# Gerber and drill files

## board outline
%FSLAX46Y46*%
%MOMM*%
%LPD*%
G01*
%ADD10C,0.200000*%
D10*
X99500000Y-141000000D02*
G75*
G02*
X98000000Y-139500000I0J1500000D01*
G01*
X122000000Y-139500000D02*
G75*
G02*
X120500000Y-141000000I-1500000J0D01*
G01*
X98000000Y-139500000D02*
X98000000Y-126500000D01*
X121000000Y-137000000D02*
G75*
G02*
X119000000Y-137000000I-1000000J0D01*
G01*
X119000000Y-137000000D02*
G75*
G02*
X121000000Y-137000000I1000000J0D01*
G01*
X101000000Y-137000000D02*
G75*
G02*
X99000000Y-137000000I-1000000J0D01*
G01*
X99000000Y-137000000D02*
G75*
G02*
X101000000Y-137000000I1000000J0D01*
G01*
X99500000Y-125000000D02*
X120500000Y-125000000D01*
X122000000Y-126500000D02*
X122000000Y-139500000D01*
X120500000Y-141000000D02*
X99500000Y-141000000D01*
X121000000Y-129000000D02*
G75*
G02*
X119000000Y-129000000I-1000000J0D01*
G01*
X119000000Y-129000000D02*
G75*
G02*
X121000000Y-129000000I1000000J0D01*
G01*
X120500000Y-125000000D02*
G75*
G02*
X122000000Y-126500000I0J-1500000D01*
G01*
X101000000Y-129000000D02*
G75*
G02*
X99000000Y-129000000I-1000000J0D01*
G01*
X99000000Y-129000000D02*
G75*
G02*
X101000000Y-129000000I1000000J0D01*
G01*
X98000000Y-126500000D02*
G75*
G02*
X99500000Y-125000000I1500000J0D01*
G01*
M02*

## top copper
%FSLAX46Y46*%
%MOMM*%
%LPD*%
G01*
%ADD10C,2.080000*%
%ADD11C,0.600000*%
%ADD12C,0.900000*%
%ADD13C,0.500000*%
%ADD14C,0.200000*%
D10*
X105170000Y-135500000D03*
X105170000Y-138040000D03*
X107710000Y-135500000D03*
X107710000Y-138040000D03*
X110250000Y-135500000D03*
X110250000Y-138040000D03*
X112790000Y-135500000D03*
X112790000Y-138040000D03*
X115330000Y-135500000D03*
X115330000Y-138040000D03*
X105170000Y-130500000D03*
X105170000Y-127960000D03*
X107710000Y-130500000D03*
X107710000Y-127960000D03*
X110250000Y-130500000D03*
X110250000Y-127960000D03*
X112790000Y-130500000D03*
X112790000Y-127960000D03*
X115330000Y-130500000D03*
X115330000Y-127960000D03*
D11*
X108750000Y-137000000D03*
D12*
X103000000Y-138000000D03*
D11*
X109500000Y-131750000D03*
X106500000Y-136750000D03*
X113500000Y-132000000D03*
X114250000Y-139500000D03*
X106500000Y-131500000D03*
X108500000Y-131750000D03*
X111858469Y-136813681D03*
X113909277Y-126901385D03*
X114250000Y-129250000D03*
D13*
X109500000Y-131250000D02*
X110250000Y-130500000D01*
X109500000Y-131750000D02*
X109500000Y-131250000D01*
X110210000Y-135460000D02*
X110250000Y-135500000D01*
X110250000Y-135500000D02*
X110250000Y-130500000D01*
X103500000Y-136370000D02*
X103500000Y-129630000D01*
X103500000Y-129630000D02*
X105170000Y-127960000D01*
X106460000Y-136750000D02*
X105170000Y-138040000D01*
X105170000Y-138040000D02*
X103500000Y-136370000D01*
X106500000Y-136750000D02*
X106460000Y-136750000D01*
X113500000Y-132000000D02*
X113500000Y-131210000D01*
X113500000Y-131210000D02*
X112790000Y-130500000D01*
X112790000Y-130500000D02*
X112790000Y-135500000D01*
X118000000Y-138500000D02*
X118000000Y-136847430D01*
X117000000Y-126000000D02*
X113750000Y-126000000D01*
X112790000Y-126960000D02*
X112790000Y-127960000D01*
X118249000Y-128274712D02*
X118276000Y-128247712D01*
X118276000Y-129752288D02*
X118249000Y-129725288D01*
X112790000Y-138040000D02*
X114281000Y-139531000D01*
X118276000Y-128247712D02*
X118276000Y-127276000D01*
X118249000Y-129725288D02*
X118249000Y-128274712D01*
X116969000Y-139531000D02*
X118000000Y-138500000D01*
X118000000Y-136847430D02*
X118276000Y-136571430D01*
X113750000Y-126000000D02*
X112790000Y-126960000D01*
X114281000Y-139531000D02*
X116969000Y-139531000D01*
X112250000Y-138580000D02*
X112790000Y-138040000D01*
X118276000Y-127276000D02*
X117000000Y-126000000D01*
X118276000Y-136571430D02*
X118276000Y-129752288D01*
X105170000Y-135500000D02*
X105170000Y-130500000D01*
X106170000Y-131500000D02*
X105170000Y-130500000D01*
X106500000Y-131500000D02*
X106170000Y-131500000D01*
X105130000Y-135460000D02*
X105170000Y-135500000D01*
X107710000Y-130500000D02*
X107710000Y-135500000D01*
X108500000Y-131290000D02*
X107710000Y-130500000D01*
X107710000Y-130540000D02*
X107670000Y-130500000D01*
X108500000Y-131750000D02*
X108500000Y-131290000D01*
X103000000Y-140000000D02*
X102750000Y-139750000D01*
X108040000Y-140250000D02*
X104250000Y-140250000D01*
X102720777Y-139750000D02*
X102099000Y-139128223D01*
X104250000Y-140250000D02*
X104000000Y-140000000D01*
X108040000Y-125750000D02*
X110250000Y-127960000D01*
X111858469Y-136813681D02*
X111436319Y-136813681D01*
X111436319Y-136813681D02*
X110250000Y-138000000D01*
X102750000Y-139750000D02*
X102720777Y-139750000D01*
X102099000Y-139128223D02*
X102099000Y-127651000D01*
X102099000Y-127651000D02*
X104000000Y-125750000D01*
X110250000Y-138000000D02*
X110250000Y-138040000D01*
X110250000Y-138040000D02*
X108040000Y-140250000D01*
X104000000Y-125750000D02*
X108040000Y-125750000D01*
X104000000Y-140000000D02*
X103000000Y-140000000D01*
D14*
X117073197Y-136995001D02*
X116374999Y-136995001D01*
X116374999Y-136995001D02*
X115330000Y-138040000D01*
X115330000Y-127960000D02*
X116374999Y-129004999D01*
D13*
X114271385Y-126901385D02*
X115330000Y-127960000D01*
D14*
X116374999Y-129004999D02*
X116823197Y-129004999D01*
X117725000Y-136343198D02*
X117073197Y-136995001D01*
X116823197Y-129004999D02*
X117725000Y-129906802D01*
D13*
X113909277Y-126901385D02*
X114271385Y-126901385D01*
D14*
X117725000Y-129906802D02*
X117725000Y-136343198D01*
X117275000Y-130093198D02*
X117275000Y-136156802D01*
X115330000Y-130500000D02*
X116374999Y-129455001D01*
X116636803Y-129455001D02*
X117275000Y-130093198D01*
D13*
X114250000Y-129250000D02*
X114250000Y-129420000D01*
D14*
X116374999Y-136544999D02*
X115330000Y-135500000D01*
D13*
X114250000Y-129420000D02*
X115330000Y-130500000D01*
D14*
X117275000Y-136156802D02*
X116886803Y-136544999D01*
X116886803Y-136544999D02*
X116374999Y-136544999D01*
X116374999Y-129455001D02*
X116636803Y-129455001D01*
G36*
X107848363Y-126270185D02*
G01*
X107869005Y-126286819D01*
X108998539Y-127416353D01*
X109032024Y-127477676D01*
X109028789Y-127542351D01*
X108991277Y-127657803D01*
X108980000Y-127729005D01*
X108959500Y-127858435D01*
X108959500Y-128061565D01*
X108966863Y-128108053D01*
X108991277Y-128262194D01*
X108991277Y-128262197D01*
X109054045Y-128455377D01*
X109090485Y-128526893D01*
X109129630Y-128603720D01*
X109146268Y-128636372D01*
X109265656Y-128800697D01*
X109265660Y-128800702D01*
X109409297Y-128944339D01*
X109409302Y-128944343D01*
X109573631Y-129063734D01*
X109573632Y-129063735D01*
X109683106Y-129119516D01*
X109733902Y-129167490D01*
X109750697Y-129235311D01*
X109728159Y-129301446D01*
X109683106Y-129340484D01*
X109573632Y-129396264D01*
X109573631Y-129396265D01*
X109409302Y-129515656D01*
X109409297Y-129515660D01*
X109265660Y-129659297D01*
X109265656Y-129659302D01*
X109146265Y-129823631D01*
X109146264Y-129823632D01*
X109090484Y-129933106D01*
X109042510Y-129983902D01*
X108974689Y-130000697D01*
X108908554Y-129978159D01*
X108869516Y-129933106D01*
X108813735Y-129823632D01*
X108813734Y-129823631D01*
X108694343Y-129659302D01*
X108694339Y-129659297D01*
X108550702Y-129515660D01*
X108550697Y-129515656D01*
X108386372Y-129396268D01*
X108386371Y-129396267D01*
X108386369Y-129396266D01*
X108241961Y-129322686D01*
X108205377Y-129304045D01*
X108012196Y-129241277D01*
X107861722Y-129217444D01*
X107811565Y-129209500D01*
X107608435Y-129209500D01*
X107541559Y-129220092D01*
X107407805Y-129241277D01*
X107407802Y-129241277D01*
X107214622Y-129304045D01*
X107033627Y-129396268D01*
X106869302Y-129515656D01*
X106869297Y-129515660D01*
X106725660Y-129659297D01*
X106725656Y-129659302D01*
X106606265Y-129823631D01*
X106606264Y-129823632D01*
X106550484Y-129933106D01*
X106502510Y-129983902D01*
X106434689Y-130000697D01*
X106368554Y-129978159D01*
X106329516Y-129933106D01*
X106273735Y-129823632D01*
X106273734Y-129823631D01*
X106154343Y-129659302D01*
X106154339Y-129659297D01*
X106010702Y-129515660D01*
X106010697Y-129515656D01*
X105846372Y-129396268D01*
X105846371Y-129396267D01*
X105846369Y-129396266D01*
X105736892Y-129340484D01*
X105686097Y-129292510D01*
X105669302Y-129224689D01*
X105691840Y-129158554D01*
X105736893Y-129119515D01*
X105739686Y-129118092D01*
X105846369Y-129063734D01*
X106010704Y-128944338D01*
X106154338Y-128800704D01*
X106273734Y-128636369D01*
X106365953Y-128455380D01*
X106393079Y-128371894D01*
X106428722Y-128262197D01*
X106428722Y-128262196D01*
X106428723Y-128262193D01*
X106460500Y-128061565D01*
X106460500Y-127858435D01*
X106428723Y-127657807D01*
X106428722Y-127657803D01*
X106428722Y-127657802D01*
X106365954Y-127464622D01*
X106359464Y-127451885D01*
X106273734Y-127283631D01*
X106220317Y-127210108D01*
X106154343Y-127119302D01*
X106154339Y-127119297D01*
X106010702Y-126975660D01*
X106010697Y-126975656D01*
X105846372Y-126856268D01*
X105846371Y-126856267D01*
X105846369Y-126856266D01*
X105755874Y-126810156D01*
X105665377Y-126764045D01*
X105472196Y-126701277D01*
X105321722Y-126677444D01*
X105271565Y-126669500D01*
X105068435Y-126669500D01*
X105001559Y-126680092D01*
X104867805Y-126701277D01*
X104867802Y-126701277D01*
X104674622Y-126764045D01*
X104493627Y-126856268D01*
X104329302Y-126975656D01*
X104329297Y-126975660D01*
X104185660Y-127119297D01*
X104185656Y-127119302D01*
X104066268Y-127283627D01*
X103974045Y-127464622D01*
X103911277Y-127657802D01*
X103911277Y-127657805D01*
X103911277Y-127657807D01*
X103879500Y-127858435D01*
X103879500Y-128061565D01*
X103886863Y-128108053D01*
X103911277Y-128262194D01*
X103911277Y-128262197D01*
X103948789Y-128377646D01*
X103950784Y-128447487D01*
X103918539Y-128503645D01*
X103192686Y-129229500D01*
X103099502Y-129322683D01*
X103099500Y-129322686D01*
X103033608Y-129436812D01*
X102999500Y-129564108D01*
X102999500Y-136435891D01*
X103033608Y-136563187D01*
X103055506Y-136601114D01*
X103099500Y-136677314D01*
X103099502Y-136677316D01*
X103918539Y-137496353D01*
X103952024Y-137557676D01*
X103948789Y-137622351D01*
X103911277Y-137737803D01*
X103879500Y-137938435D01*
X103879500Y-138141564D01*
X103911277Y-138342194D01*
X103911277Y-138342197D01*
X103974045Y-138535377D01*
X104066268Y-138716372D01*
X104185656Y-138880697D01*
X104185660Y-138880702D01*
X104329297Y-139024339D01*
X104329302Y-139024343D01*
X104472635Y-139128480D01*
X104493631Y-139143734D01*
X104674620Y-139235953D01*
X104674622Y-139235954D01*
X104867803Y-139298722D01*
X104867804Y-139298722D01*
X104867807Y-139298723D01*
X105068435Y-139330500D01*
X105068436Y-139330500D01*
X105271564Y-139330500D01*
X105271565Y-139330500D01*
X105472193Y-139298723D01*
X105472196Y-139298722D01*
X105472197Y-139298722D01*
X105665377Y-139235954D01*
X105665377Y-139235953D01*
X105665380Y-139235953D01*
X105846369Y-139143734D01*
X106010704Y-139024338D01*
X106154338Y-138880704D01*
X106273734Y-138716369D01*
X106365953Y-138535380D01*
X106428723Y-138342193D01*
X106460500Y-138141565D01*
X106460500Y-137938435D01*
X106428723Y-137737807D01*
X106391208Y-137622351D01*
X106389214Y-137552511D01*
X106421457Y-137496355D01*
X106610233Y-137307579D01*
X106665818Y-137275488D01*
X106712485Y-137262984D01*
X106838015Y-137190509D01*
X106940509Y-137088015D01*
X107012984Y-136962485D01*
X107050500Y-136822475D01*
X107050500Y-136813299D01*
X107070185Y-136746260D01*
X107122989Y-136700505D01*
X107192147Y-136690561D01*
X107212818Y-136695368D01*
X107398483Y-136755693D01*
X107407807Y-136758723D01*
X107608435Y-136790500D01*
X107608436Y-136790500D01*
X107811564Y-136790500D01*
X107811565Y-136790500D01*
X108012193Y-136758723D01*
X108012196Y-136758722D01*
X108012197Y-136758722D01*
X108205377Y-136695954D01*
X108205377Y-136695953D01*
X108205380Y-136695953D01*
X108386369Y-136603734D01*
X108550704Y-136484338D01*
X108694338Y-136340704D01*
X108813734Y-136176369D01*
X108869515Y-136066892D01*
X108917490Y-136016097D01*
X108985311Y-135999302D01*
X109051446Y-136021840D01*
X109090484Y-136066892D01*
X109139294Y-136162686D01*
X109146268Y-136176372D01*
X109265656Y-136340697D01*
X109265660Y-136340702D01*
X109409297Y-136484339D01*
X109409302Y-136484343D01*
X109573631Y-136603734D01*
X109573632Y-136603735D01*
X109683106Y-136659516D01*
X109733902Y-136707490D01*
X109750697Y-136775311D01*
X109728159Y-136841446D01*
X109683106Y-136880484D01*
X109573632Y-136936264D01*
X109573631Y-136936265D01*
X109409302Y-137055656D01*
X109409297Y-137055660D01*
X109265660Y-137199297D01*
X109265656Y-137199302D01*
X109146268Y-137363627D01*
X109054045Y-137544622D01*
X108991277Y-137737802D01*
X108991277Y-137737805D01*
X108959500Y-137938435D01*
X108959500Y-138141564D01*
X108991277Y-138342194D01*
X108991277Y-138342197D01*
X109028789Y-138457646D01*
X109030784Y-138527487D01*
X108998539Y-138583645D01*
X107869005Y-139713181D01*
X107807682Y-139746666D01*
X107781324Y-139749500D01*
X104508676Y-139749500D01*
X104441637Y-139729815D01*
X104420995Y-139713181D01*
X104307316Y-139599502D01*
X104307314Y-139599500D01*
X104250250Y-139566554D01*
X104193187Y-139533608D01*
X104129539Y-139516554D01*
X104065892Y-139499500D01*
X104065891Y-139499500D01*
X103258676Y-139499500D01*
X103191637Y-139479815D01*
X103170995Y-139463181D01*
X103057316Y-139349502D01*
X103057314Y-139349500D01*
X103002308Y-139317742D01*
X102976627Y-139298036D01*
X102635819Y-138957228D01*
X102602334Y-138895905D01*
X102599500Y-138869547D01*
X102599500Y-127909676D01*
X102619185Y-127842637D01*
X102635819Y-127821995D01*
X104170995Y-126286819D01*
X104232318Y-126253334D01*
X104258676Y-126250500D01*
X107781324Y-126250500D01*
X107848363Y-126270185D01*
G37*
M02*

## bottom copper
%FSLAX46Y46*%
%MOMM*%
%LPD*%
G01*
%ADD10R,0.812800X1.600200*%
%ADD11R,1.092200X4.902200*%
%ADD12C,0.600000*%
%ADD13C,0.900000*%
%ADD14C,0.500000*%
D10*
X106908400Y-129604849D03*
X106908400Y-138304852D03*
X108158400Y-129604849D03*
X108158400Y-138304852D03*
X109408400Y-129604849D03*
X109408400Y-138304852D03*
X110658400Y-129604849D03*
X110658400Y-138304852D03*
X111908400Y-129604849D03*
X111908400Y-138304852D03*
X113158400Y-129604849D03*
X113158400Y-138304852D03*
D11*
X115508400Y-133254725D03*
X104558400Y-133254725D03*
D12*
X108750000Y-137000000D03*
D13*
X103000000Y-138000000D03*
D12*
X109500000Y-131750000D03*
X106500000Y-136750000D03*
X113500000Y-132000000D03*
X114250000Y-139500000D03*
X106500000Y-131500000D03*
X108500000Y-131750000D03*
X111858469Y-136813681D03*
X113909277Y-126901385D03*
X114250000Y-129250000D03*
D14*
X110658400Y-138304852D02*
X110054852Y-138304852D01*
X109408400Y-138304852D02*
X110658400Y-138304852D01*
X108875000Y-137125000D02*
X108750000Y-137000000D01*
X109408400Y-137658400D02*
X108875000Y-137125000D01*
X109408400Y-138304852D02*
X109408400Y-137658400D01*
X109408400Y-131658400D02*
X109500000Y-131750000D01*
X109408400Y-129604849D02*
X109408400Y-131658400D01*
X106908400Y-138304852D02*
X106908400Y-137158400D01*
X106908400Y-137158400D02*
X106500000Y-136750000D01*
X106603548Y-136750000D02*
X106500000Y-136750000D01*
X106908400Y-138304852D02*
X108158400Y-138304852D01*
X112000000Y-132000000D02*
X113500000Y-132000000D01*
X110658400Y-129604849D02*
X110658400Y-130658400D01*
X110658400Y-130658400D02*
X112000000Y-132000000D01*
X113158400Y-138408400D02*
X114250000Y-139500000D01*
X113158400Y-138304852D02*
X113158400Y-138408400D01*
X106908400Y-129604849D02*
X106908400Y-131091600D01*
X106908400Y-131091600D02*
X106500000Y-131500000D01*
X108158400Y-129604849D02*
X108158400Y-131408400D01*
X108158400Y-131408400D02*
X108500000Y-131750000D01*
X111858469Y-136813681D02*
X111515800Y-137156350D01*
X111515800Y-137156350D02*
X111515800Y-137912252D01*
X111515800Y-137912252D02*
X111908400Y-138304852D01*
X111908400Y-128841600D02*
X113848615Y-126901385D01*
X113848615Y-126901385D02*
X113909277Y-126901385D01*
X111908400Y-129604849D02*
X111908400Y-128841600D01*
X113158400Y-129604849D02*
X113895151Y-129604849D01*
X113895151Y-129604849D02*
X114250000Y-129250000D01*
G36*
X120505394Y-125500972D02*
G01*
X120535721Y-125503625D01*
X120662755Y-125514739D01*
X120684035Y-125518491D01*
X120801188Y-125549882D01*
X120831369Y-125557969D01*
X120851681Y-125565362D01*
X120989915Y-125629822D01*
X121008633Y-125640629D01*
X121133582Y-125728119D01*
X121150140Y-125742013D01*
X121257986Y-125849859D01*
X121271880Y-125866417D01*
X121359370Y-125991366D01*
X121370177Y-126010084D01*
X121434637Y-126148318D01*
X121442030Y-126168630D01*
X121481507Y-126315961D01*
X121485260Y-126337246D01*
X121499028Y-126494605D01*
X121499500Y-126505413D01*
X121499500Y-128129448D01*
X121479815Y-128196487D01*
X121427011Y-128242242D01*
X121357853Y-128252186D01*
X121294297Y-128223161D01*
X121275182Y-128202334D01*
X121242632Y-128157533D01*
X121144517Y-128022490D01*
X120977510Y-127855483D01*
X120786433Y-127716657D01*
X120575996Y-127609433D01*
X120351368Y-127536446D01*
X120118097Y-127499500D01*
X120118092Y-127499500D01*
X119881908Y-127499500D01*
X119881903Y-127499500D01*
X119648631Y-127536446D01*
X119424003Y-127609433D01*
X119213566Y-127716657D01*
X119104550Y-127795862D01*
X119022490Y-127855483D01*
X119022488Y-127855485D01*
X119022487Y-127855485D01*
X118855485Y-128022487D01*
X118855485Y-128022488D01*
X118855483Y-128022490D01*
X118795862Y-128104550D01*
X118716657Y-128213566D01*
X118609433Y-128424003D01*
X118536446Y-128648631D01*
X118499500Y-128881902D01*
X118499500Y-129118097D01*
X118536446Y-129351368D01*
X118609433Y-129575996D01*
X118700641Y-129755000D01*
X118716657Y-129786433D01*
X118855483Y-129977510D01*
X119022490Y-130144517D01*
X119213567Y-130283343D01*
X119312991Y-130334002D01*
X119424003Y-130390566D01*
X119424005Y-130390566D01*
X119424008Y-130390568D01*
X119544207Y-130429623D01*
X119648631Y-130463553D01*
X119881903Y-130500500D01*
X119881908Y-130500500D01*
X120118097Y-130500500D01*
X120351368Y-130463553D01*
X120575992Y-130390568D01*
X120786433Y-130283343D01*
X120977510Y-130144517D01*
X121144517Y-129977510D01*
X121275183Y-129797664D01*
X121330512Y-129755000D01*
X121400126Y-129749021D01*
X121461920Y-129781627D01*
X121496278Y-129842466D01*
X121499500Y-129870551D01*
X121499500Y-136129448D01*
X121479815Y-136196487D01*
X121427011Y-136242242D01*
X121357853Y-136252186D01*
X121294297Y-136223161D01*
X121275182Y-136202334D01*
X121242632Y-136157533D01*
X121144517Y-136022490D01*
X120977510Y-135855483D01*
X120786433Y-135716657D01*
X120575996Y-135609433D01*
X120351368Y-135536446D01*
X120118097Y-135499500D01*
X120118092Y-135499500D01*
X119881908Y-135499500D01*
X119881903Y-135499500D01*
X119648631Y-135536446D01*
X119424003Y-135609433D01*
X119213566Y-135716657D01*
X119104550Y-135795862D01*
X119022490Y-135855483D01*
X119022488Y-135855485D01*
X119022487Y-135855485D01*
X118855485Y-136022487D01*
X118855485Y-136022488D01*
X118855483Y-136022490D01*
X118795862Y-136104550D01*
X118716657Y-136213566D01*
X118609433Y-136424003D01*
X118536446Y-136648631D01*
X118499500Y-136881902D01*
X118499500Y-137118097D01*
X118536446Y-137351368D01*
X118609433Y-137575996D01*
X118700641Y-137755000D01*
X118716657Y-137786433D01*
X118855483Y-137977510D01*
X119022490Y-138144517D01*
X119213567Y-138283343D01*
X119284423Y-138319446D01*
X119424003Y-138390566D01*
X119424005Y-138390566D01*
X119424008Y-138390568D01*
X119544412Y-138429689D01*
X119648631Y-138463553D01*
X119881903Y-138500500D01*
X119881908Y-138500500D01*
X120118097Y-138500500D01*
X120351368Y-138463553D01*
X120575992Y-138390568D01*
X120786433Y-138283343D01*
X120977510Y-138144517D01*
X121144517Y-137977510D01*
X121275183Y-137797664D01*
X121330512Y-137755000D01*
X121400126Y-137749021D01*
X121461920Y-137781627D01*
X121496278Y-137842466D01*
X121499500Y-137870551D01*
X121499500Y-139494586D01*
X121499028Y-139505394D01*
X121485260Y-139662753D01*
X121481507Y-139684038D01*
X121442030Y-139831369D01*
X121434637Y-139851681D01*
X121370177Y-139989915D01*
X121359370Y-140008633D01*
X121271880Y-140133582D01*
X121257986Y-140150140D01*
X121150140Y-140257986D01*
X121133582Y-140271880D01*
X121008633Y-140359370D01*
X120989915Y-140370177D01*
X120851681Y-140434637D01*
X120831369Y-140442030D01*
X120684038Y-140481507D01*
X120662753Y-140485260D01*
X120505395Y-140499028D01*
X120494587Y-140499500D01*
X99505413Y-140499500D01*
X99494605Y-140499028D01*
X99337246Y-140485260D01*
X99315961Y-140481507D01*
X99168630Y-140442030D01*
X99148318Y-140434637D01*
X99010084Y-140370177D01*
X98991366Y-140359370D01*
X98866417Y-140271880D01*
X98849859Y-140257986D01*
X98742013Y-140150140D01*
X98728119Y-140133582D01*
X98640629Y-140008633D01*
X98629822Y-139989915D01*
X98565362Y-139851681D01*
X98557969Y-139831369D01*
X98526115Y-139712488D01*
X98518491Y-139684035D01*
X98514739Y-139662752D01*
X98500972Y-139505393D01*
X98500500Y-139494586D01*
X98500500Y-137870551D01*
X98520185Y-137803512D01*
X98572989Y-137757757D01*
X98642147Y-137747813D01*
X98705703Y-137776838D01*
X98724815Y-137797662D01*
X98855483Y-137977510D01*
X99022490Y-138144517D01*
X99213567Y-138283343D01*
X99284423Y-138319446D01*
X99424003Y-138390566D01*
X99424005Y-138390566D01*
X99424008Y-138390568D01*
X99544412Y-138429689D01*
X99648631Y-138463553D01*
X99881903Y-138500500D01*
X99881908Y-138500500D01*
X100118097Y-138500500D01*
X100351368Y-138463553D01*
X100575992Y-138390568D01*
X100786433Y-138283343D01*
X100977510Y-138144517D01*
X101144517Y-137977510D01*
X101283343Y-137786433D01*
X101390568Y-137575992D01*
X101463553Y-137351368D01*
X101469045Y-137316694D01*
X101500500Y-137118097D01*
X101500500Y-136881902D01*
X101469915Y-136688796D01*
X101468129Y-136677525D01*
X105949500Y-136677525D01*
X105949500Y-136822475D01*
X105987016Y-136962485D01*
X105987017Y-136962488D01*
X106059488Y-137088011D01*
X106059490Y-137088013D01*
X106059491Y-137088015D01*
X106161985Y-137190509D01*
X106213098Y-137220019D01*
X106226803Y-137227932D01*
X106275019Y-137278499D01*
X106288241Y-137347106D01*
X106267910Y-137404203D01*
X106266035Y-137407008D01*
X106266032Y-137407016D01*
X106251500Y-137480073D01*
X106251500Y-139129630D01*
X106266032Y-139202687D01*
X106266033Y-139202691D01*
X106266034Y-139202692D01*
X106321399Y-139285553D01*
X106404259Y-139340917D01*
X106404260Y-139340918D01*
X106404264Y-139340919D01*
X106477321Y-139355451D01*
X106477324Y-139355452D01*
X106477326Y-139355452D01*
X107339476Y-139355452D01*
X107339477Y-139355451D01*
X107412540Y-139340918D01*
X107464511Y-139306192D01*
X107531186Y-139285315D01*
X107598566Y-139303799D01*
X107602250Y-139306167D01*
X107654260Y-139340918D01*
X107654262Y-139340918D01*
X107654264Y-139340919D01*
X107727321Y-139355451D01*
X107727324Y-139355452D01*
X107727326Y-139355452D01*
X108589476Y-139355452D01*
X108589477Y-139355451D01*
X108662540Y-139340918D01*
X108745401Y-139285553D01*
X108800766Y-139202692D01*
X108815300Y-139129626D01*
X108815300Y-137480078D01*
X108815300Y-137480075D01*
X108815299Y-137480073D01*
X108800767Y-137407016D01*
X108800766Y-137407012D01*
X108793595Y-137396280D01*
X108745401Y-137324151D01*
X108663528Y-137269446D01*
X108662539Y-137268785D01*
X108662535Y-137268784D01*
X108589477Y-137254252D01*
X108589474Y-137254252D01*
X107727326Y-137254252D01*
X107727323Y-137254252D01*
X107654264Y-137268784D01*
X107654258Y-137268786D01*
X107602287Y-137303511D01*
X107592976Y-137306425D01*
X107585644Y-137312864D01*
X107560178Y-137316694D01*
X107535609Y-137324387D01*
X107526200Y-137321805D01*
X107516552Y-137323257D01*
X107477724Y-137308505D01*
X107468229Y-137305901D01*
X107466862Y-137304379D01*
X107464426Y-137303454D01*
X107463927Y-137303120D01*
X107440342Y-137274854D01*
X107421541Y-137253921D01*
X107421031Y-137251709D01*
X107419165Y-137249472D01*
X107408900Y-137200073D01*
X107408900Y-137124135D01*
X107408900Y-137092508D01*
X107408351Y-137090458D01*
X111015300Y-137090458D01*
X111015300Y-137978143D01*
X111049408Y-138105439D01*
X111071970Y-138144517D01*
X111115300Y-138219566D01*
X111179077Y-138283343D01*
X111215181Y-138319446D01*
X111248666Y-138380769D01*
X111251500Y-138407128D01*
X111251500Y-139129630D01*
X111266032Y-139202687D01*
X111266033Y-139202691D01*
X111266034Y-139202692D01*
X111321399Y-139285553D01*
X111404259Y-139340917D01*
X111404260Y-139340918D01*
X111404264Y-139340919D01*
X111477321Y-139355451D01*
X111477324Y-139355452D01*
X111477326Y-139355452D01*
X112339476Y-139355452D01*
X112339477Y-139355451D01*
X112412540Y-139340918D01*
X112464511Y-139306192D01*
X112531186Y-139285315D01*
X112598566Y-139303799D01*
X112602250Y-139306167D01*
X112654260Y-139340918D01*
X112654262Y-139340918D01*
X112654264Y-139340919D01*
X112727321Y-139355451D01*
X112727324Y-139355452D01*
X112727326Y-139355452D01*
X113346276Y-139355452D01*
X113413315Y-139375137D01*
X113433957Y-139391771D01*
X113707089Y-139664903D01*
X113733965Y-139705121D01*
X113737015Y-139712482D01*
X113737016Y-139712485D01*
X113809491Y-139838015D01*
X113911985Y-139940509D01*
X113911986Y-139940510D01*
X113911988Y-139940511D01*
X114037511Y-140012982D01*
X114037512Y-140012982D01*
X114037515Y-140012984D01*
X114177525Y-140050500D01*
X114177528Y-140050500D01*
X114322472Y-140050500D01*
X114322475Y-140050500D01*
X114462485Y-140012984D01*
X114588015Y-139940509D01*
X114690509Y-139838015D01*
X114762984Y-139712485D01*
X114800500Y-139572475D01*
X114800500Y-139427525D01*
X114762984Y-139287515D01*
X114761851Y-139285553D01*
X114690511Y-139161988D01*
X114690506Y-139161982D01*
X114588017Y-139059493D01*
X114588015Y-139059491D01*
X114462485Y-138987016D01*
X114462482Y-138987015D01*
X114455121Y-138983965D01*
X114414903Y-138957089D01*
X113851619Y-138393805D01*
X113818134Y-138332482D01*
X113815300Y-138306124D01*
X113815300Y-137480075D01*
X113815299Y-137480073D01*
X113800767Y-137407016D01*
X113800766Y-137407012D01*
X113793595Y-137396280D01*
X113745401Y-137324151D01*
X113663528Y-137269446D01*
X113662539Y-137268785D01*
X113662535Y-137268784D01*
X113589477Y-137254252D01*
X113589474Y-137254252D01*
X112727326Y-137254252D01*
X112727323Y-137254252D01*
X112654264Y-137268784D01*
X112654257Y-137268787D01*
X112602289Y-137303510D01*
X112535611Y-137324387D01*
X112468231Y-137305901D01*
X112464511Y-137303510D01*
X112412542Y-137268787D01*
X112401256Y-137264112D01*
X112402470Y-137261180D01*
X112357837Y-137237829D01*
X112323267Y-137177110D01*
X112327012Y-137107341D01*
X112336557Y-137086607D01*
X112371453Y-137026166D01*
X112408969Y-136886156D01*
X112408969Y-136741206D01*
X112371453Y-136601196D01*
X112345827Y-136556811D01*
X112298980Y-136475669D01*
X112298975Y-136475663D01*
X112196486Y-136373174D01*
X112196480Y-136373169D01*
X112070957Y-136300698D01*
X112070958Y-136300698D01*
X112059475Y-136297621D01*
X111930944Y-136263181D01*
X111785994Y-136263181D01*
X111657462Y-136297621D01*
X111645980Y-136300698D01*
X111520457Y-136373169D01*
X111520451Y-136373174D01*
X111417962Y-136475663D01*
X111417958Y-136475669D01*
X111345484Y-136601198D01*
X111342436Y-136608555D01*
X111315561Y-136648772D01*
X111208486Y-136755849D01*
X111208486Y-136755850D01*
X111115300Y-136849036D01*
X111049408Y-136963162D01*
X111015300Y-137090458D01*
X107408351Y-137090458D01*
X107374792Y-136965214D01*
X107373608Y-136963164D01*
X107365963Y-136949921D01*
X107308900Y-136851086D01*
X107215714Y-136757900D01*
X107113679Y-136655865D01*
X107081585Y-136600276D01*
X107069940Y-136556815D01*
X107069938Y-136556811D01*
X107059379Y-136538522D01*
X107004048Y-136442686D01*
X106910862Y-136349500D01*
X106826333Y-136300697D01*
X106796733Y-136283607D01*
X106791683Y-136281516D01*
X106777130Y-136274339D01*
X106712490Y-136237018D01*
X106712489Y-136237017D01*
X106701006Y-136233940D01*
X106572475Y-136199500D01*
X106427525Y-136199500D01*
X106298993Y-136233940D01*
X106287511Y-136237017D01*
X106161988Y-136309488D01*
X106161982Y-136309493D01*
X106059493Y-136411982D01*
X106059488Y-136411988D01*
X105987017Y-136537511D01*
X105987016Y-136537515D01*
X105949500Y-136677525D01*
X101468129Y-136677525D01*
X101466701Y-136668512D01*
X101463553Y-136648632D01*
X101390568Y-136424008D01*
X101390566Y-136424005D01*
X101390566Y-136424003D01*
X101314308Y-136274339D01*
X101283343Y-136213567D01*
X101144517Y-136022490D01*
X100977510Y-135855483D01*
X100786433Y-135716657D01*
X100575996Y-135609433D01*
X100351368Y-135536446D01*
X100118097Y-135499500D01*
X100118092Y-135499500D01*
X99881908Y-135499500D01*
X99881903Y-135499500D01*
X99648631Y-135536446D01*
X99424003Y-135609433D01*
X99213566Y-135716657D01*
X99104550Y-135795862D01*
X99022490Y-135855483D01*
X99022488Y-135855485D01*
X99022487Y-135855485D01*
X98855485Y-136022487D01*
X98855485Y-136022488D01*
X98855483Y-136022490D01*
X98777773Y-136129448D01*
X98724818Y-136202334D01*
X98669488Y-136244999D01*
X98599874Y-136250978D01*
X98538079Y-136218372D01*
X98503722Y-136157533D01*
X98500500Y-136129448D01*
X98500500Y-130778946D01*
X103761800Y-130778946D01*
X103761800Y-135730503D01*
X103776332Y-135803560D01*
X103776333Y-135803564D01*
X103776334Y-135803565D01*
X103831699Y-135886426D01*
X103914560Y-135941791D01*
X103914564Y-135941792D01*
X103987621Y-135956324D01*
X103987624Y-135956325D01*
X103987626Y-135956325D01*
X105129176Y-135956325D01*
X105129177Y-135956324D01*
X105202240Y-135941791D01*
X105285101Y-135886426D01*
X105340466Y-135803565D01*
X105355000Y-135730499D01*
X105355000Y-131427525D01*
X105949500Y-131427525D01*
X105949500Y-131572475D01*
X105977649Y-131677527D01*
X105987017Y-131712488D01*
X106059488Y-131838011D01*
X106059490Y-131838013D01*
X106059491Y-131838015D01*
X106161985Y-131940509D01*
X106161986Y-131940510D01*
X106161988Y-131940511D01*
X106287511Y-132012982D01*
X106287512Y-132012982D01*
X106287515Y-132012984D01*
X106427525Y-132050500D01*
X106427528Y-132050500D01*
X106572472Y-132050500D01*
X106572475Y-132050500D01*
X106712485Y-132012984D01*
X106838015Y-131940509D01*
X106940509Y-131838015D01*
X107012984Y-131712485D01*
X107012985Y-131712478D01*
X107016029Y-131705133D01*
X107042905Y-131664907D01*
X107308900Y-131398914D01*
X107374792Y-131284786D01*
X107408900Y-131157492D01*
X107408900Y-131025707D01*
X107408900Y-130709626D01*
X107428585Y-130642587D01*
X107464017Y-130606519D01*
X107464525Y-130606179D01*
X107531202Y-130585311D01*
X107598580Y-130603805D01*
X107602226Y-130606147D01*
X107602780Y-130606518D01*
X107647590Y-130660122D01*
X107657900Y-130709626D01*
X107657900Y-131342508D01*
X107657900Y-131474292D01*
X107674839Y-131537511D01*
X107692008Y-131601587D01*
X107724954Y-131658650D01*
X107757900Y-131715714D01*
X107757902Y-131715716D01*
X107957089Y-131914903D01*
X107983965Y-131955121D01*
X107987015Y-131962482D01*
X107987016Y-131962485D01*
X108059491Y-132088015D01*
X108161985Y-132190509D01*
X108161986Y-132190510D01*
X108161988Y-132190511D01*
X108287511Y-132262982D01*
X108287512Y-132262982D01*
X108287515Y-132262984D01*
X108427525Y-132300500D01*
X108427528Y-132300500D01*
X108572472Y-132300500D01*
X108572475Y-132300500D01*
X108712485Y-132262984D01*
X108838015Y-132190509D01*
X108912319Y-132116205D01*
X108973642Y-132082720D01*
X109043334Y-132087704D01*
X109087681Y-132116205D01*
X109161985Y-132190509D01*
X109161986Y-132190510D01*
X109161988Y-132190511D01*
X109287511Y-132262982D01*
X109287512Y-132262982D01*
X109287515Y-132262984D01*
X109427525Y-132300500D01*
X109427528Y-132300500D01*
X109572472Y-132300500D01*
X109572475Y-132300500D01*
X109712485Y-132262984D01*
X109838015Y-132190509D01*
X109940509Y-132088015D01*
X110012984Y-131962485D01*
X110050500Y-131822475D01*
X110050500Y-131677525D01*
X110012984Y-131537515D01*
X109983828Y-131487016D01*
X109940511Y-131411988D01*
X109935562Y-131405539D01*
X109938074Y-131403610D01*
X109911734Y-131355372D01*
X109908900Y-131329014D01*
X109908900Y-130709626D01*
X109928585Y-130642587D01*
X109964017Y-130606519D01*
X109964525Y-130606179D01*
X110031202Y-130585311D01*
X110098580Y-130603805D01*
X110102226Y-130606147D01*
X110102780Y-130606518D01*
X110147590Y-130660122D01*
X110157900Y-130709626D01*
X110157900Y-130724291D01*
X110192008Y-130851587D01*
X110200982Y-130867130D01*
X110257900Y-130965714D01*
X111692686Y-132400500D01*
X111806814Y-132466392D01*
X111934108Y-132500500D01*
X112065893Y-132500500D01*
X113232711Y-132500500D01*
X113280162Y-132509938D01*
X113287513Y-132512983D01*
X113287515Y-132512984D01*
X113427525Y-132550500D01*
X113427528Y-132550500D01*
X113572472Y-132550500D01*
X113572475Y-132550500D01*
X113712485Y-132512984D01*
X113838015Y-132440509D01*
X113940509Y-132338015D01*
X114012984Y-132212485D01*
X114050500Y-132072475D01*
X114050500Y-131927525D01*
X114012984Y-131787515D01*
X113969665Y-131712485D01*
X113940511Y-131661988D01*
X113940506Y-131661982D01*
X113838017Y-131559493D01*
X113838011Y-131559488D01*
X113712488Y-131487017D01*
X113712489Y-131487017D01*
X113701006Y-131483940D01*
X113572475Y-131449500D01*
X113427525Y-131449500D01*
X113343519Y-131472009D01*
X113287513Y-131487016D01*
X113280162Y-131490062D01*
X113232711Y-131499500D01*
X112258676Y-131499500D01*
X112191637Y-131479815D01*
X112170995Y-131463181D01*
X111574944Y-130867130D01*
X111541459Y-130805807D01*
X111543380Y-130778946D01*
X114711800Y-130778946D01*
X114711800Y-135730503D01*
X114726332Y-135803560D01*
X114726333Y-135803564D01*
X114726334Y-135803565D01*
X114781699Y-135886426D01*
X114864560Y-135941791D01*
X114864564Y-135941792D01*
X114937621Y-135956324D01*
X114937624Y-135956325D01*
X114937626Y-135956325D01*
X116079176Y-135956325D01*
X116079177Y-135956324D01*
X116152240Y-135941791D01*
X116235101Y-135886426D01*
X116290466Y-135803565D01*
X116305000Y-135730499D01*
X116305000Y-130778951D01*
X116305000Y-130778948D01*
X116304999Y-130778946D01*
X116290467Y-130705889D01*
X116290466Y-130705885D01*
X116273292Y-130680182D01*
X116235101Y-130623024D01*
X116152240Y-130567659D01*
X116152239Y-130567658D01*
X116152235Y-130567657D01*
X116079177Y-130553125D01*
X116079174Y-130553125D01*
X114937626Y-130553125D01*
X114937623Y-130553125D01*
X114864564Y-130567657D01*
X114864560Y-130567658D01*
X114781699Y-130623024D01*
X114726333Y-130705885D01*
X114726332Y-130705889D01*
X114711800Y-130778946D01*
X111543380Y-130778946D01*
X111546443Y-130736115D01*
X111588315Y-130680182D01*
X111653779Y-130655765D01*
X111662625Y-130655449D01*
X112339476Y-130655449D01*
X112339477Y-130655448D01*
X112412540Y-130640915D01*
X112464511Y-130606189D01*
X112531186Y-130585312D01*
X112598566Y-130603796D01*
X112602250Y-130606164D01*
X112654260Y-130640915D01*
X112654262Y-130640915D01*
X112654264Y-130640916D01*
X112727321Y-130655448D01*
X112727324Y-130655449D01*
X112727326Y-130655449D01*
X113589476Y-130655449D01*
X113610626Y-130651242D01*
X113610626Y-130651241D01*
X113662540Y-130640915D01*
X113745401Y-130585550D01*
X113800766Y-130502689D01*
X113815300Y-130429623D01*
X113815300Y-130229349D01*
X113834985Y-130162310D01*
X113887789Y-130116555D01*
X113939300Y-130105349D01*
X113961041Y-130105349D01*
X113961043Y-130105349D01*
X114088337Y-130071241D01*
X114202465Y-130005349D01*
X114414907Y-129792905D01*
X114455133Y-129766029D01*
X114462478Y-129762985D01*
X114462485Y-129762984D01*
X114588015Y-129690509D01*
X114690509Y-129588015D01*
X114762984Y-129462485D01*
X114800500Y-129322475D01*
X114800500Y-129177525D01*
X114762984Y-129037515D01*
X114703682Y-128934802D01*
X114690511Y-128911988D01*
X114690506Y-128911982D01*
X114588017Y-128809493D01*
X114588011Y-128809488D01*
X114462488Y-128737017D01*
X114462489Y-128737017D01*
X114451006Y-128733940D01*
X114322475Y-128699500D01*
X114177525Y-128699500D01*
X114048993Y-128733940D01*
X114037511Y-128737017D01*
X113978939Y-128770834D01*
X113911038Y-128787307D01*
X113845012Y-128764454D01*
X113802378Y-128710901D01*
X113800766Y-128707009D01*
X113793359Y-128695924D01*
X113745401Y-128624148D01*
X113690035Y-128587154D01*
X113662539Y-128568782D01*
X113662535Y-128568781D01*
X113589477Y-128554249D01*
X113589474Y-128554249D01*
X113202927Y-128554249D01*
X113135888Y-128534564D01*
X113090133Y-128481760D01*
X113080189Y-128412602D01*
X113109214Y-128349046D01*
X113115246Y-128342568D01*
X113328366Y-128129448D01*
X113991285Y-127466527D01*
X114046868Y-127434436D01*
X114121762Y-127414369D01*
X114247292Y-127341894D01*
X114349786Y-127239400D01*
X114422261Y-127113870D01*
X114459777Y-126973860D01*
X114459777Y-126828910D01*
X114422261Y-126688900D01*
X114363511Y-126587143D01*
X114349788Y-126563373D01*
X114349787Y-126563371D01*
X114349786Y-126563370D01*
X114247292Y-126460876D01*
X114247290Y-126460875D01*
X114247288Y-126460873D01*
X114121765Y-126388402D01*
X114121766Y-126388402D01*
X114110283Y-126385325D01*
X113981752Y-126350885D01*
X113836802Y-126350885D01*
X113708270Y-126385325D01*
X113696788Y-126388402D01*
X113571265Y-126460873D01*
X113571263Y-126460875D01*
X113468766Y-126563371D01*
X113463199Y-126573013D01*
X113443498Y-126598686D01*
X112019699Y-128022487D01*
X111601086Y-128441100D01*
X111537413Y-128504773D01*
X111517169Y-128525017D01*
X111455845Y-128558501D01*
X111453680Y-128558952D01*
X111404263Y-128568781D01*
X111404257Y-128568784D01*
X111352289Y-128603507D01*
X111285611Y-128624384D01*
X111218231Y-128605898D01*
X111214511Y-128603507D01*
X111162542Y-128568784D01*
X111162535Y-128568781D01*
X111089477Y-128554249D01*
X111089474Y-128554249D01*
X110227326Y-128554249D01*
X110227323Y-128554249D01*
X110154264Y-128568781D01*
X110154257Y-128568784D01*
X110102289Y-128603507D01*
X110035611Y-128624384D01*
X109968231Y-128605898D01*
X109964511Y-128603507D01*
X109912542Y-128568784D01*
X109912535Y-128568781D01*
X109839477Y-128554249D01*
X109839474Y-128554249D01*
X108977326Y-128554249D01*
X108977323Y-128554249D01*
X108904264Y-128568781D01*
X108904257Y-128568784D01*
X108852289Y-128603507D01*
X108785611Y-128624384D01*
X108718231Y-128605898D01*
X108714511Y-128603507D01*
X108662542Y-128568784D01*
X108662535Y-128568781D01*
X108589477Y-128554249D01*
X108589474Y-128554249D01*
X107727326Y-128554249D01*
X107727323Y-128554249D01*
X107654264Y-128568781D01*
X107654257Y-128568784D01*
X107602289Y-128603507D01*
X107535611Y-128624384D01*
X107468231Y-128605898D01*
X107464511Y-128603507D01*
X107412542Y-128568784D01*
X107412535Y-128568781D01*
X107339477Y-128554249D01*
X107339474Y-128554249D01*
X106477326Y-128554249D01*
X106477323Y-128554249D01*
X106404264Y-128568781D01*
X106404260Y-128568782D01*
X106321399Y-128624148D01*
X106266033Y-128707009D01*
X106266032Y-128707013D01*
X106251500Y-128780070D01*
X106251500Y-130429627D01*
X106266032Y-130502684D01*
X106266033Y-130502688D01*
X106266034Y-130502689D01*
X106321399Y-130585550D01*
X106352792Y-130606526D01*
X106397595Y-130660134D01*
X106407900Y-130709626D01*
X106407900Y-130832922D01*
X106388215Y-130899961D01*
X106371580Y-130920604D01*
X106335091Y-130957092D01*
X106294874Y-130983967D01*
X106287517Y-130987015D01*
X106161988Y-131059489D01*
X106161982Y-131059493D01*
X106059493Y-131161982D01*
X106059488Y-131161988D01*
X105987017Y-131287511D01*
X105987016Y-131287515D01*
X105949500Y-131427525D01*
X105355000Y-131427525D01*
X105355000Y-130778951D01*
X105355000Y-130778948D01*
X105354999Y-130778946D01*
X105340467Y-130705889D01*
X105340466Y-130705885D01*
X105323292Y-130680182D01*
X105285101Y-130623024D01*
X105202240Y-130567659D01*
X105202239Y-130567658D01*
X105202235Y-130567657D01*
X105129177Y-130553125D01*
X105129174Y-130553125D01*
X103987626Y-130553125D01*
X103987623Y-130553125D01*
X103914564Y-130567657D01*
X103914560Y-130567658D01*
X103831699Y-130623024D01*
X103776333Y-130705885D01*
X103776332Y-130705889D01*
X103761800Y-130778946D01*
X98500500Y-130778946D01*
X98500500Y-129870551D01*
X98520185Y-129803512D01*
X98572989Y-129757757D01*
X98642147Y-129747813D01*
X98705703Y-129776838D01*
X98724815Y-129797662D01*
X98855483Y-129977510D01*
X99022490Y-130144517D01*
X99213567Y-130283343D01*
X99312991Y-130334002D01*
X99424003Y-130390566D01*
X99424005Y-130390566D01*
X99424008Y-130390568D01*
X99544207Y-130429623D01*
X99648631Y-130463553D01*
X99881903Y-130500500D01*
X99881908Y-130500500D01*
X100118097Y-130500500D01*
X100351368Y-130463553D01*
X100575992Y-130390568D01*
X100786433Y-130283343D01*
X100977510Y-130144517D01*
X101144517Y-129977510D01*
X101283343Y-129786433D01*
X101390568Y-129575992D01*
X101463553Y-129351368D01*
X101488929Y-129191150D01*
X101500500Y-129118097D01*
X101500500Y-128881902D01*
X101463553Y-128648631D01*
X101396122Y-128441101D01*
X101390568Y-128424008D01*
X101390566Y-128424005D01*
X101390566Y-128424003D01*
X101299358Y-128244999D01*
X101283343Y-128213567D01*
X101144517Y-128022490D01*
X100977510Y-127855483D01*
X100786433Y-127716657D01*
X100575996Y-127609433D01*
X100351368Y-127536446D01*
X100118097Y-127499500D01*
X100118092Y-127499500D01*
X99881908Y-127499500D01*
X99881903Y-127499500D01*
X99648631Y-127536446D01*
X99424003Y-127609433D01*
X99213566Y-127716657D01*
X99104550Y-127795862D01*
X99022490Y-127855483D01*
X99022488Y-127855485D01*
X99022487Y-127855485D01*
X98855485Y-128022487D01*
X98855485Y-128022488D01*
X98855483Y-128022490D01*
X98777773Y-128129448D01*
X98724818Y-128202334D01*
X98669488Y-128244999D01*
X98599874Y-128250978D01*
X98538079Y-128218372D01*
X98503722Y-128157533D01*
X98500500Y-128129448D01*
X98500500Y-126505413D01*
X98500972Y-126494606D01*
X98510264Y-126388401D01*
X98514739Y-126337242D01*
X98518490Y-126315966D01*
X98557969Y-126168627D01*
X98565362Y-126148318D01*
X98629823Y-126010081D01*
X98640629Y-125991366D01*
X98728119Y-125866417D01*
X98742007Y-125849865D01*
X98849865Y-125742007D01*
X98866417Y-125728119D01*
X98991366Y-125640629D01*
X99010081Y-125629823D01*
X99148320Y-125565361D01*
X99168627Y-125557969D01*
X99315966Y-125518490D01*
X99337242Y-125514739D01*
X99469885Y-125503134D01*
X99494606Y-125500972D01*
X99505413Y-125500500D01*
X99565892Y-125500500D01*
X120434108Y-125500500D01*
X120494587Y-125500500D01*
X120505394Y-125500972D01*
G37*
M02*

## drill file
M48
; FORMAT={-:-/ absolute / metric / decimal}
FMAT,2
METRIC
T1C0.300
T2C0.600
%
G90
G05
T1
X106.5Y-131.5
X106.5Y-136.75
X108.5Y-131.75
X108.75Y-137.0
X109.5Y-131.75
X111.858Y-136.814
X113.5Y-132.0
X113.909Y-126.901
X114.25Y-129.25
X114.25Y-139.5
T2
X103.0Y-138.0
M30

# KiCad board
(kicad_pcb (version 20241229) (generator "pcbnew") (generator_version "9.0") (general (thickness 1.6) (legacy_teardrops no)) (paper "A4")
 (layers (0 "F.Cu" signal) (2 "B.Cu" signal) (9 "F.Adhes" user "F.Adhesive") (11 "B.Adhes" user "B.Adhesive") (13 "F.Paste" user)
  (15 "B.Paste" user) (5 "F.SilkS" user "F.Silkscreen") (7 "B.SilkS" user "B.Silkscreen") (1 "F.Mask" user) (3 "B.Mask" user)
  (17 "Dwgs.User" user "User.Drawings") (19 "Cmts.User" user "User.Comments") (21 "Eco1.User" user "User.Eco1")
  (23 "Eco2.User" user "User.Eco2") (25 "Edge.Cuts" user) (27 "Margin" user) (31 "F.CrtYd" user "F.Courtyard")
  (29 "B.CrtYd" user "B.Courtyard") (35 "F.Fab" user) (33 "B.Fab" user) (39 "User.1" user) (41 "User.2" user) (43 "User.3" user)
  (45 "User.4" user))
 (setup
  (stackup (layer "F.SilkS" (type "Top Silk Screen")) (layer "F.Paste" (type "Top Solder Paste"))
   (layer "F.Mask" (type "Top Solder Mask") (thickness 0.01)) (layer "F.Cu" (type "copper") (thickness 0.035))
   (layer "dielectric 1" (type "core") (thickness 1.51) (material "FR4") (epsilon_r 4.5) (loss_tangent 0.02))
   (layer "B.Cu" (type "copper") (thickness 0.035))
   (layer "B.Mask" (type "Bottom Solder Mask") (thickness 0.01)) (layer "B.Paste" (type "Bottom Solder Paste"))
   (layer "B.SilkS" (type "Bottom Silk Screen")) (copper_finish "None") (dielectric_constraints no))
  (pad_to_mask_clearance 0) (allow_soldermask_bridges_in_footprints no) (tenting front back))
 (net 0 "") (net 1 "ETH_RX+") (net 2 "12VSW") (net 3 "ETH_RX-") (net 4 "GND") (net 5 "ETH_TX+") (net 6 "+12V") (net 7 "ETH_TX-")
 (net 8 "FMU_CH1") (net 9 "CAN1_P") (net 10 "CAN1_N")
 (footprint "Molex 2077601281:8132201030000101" (layer "F.Cu") (at 110.25 136.54)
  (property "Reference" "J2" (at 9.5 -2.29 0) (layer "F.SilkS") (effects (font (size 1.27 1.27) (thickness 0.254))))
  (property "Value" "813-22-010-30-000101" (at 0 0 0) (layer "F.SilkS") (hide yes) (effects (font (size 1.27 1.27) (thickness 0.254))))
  (pad "1" smd circle (at -5.08 -1.04 270) (size 2.08 2.08) (layers "F.Cu" "F.Mask" "F.Paste") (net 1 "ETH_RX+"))
  (pad "2" smd circle (at -5.08 1.5 270) (size 2.08 2.08) (layers "F.Cu" "F.Mask" "F.Paste") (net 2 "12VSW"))
  (pad "3" smd circle (at -2.54 -1.04 270) (size 2.08 2.08) (layers "F.Cu" "F.Mask" "F.Paste") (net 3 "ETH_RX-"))
  (pad "4" smd circle (at -2.54 1.5 270) (size 2.08 2.08) (layers "F.Cu" "F.Mask" "F.Paste") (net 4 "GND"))
  (pad "5" smd circle (at 0 -1.04 270) (size 2.08 2.08) (layers "F.Cu" "F.Mask" "F.Paste") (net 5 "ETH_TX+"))
  (pad "6" smd circle (at 0 1.5 270) (size 2.08 2.08) (layers "F.Cu" "F.Mask" "F.Paste") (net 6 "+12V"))
  (pad "7" smd circle (at 2.54 -1.04 270) (size 2.08 2.08) (layers "F.Cu" "F.Mask" "F.Paste") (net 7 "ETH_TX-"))
  (pad "8" smd circle (at 2.54 1.5 270) (size 2.08 2.08) (layers "F.Cu" "F.Mask" "F.Paste") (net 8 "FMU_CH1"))
  (pad "9" smd circle (at 5.08 -1.04 270) (size 2.08 2.08) (layers "F.Cu" "F.Mask" "F.Paste") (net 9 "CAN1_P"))
  (pad "10" smd circle (at 5.08 1.5 270) (size 2.08 2.08) (layers "F.Cu" "F.Mask" "F.Paste") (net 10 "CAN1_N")))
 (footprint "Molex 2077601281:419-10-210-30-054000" (layer "F.Cu") (at 110.25 129)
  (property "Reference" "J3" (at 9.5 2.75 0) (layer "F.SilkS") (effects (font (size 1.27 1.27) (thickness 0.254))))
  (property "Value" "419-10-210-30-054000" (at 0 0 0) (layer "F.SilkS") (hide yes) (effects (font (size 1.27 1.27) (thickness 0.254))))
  (pad "1" smd circle (at -5.08 1.5 90) (size 2.08 2.08) (layers "F.Cu" "F.Mask" "F.Paste") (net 1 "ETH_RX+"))
  (pad "2" smd circle (at -5.08 -1.04 90) (size 2.08 2.08) (layers "F.Cu" "F.Mask" "F.Paste") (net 2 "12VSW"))
  (pad "3" smd circle (at -2.54 1.5 90) (size 2.08 2.08) (layers "F.Cu" "F.Mask" "F.Paste") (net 3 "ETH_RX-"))
  (pad "4" smd circle (at -2.54 -1.04 90) (size 2.08 2.08) (layers "F.Cu" "F.Mask" "F.Paste") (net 4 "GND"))
  (pad "5" smd circle (at 0 1.5 90) (size 2.08 2.08) (layers "F.Cu" "F.Mask" "F.Paste") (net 5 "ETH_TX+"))
  (pad "6" smd circle (at 0 -1.04 90) (size 2.08 2.08) (layers "F.Cu" "F.Mask" "F.Paste") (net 6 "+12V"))
  (pad "7" smd circle (at 2.54 1.5 90) (size 2.08 2.08) (layers "F.Cu" "F.Mask" "F.Paste") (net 7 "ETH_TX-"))
  (pad "8" smd circle (at 2.54 -1.04 90) (size 2.08 2.08) (layers "F.Cu" "F.Mask" "F.Paste") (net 8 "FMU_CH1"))
  (pad "9" smd circle (at 5.08 1.5 90) (size 2.08 2.08) (layers "F.Cu" "F.Mask" "F.Paste") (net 9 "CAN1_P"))
  (pad "10" smd circle (at 5.08 -1.04 90) (size 2.08 2.08) (layers "F.Cu" "F.Mask" "F.Paste") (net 10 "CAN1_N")))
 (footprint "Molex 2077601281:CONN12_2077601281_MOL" (layer "B.Cu") (at 110.0334 133.958551 180)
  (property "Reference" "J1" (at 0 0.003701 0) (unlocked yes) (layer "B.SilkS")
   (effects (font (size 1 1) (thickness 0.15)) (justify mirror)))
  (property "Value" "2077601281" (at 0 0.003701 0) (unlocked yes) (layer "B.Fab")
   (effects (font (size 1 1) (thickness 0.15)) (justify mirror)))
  (pad "1" smd rect (at 3.125 4.353702 180) (size 0.8128 1.6002) (layers "B.Cu" "B.Mask" "B.Paste") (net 1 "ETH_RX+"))
  (pad "2" smd rect (at 3.125 -4.346301 180) (size 0.8128 1.6002) (layers "B.Cu" "B.Mask" "B.Paste") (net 2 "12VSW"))
  (pad "3" smd rect (at 1.875 4.353702 180) (size 0.8128 1.6002) (layers "B.Cu" "B.Mask" "B.Paste") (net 3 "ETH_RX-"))
  (pad "4" smd rect (at 1.875 -4.346301 180) (size 0.8128 1.6002) (layers "B.Cu" "B.Mask" "B.Paste") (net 2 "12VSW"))
  (pad "5" smd rect (at 0.625 4.353702 180) (size 0.8128 1.6002) (layers "B.Cu" "B.Mask" "B.Paste") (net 5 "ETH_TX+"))
  (pad "6" smd rect (at 0.625 -4.346301 180) (size 0.8128 1.6002) (layers "B.Cu" "B.Mask" "B.Paste") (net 4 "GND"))
  (pad "7" smd rect (at -0.625 4.353702 180) (size 0.8128 1.6002) (layers "B.Cu" "B.Mask" "B.Paste") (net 7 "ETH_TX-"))
  (pad "8" smd rect (at -0.625 -4.346301 180) (size 0.8128 1.6002) (layers "B.Cu" "B.Mask" "B.Paste") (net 4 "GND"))
  (pad "9" smd rect (at -1.875 4.353702 180) (size 0.8128 1.6002) (layers "B.Cu" "B.Mask" "B.Paste") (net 10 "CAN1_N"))
  (pad "10" smd rect (at -1.875 -4.346301 180) (size 0.8128 1.6002) (layers "B.Cu" "B.Mask" "B.Paste") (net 6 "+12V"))
  (pad "11" smd rect (at -3.125 4.353702 180) (size 0.8128 1.6002) (layers "B.Cu" "B.Mask" "B.Paste") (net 9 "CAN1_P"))
  (pad "12" smd rect (at -3.125 -4.346301 180) (size 0.8128 1.6002) (layers "B.Cu" "B.Mask" "B.Paste") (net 8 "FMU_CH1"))
  (pad "13" smd rect (at -5.475 0.703826 180) (size 1.0922 4.9022) (layers "B.Cu" "B.Mask" "B.Paste"))
  (pad "14" smd rect (at 5.475 0.703826 180) (size 1.0922 4.9022) (layers "B.Cu" "B.Mask" "B.Paste")))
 (gr_arc (start 99.5 141) (mid 98.43934 140.56066) (end 98 139.5) (stroke (width 0.2) (type default)) (layer "Edge.Cuts"))
 (gr_arc (start 122 139.5) (mid 121.56066 140.56066) (end 120.5 141) (stroke (width 0.2) (type default)) (layer "Edge.Cuts"))
 (gr_line (start 98 139.5) (end 98 126.5) (stroke (width 0.2) (type default)) (layer "Edge.Cuts"))
 (gr_circle (center 120 137) (end 121 137) (stroke (width 0.2) (type solid)) (fill no) (layer "Edge.Cuts"))
 (gr_circle (center 100 137) (end 101 137) (stroke (width 0.2) (type solid)) (fill no) (layer "Edge.Cuts"))
 (gr_line (start 99.5 125) (end 120.5 125) (stroke (width 0.2) (type default)) (layer "Edge.Cuts"))
 (gr_line (start 122 126.5) (end 122 139.5) (stroke (width 0.2) (type default)) (layer "Edge.Cuts"))
 (gr_line (start 120.5 141) (end 99.5 141) (stroke (width 0.2) (type default)) (layer "Edge.Cuts"))
 (gr_circle (center 120 129) (end 121 129) (stroke (width 0.2) (type solid)) (fill no) (layer "Edge.Cuts"))
 (gr_arc (start 120.5 125) (mid 121.56066 125.43934) (end 122 126.5) (stroke (width 0.2) (type default)) (layer "Edge.Cuts"))
 (gr_circle (center 100 129) (end 101 129) (stroke (width 0.2) (type solid)) (fill no) (layer "Edge.Cuts"))
 (gr_arc (start 98 126.5) (mid 98.43934 125.43934) (end 99.5 125) (stroke (width 0.2) (type default)) (layer "Edge.Cuts"))
 (via (at 108.75 137) (size 0.6) (drill 0.3) (layers "F.Cu" "B.Cu") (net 4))
 (via (at 103 138) (size 0.9) (drill 0.6) (layers "F.Cu" "B.Cu") (free yes) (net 4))
 (segment (start 110.6584 138.304852) (end 110.054852 138.304852) (width 0.5) (layer "B.Cu") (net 4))
 (segment (start 109.4084 138.304852) (end 110.6584 138.304852) (width 0.5) (layer "B.Cu") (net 4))
 (segment (start 108.875 137.125) (end 108.75 137) (width 0.5) (layer "B.Cu") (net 4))
 (segment (start 109.4084 137.6584) (end 108.875 137.125) (width 0.5) (layer "B.Cu") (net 4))
 (segment (start 109.4084 138.304852) (end 109.4084 137.6584) (width 0.5) (layer "B.Cu") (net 4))
 (segment (start 109.5 131.25) (end 110.25 130.5) (width 0.5) (layer "F.Cu") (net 5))
 (segment (start 109.5 131.75) (end 109.5 131.25) (width 0.5) (layer "F.Cu") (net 5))
 (segment (start 110.21 135.46) (end 110.25 135.5) (width 0.5) (layer "F.Cu") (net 5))
 (segment (start 110.25 135.5) (end 110.25 130.5) (width 0.5) (layer "F.Cu") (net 5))
 (via (at 109.5 131.75) (size 0.6) (drill 0.3) (layers "F.Cu" "B.Cu") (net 5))
 (segment (start 109.4084 131.6584) (end 109.5 131.75) (width 0.5) (layer "B.Cu") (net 5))
 (segment (start 109.4084 129.604849) (end 109.4084 131.6584) (width 0.5) (layer "B.Cu") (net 5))
 (segment (start 103.5 136.37) (end 103.5 129.63) (width 0.5) (layer "F.Cu") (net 2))
 (segment (start 103.5 129.63) (end 105.17 127.96) (width 0.5) (layer "F.Cu") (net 2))
 (segment (start 106.46 136.75) (end 105.17 138.04) (width 0.5) (layer "F.Cu") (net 2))
 (segment (start 105.17 138.04) (end 103.5 136.37) (width 0.5) (layer "F.Cu") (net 2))
 (segment (start 106.5 136.75) (end 106.46 136.75) (width 0.5) (layer "F.Cu") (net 2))
 (via (at 106.5 136.75) (size 0.6) (drill 0.3) (layers "F.Cu" "B.Cu") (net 2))
 (segment (start 106.9084 138.304852) (end 106.9084 137.1584) (width 0.5) (layer "B.Cu") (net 2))
 (segment (start 106.9084 137.1584) (end 106.5 136.75) (width 0.5) (layer "B.Cu") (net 2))
 (segment (start 106.603548 136.75) (end 106.5 136.75) (width 0.5) (layer "B.Cu") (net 2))
 (segment (start 106.9084 138.304852) (end 108.1584 138.304852) (width 0.5) (layer "B.Cu") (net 2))
 (segment (start 113.5 132) (end 113.5 131.21) (width 0.5) (layer "F.Cu") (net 7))
 (segment (start 113.5 131.21) (end 112.79 130.5) (width 0.5) (layer "F.Cu") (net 7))
 (segment (start 112.79 130.5) (end 112.79 135.5) (width 0.5) (layer "F.Cu") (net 7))
 (via (at 113.5 132) (size 0.6) (drill 0.3) (layers "F.Cu" "B.Cu") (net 7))
 (segment (start 112 132) (end 113.5 132) (width 0.5) (layer "B.Cu") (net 7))
 (segment (start 110.6584 129.604849) (end 110.6584 130.6584) (width 0.5) (layer "B.Cu") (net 7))
 (segment (start 110.6584 130.6584) (end 112 132) (width 0.5) (layer "B.Cu") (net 7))
 (segment (start 118 138.5) (end 118 136.84743) (width 0.5) (layer "F.Cu") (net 8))
 (segment (start 117 126) (end 113.75 126) (width 0.5) (layer "F.Cu") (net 8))
 (segment (start 112.79 126.96) (end 112.79 127.96) (width 0.5) (layer "F.Cu") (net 8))
 (segment (start 118.249 128.274712) (end 118.276 128.247712) (width 0.5) (layer "F.Cu") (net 8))
 (segment (start 118.276 129.752288) (end 118.249 129.725288) (width 0.5) (layer "F.Cu") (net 8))
 (segment (start 112.79 138.04) (end 114.281 139.531) (width 0.5) (layer "F.Cu") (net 8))
 (segment (start 118.276 128.247712) (end 118.276 127.276) (width 0.5) (layer "F.Cu") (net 8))
 (segment (start 118.249 129.725288) (end 118.249 128.274712) (width 0.5) (layer "F.Cu") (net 8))
 (segment (start 116.969 139.531) (end 118 138.5) (width 0.5) (layer "F.Cu") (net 8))
 (segment (start 118 136.84743) (end 118.276 136.57143) (width 0.5) (layer "F.Cu") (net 8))
 (segment (start 113.75 126) (end 112.79 126.96) (width 0.5) (layer "F.Cu") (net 8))
 (segment (start 114.281 139.531) (end 116.969 139.531) (width 0.5) (layer "F.Cu") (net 8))
 (segment (start 112.25 138.58) (end 112.79 138.04) (width 0.5) (layer "F.Cu") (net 8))
 (segment (start 118.276 127.276) (end 117 126) (width 0.5) (layer "F.Cu") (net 8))
 (segment (start 118.276 136.57143) (end 118.276 129.752288) (width 0.5) (layer "F.Cu") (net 8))
 (via (at 114.25 139.5) (size 0.6) (drill 0.3) (layers "F.Cu" "B.Cu") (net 8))
 (segment (start 113.1584 138.4084) (end 114.25 139.5) (width 0.5) (layer "B.Cu") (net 8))
 (segment (start 113.1584 138.304852) (end 113.1584 138.4084) (width 0.5) (layer "B.Cu") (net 8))
 (segment (start 105.17 135.5) (end 105.17 130.5) (width 0.5) (layer "F.Cu") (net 1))
 (segment (start 106.17 131.5) (end 105.17 130.5) (width 0.5) (layer "F.Cu") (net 1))
 (segment (start 106.5 131.5) (end 106.17 131.5) (width 0.5) (layer "F.Cu") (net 1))
 (segment (start 105.13 135.46) (end 105.17 135.5) (width 0.5) (layer "F.Cu") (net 1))
 (via (at 106.5 131.5) (size 0.6) (drill 0.3) (layers "F.Cu" "B.Cu") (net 1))
 (segment (start 106.9084 129.604849) (end 106.9084 131.0916) (width 0.5) (layer "B.Cu") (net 1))
 (segment (start 106.9084 131.0916) (end 106.5 131.5) (width 0.5) (layer "B.Cu") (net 1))
 (segment (start 107.71 130.5) (end 107.71 135.5) (width 0.5) (layer "F.Cu") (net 3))
 (segment (start 108.5 131.29) (end 107.71 130.5) (width 0.5) (layer "F.Cu") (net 3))
 (segment (start 107.71 130.54) (end 107.67 130.5) (width 0.5) (layer "F.Cu") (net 3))
 (segment (start 108.5 131.75) (end 108.5 131.29) (width 0.5) (layer "F.Cu") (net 3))
 (via (at 108.5 131.75) (size 0.6) (drill 0.3) (layers "F.Cu" "B.Cu") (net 3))
 (segment (start 108.1584 129.604849) (end 108.1584 131.4084) (width 0.5) (layer "B.Cu") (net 3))
 (segment (start 108.1584 131.4084) (end 108.5 131.75) (width 0.5) (layer "B.Cu") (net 3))
 (segment (start 103 140) (end 102.75 139.75) (width 0.5) (layer "F.Cu") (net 6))
 (segment (start 108.04 140.25) (end 104.25 140.25) (width 0.5) (layer "F.Cu") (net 6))
 (segment (start 102.720777 139.75) (end 102.099 139.128223) (width 0.5) (layer "F.Cu") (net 6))
 (segment (start 104.25 140.25) (end 104 140) (width 0.5) (layer "F.Cu") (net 6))
 (segment (start 108.04 125.75) (end 110.25 127.96) (width 0.5) (layer "F.Cu") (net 6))
 (segment (start 111.858469 136.813681) (end 111.436319 136.813681) (width 0.5) (layer "F.Cu") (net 6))
 (segment (start 111.436319 136.813681) (end 110.25 138) (width 0.5) (layer "F.Cu") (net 6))
 (segment (start 102.75 139.75) (end 102.720777 139.75) (width 0.5) (layer "F.Cu") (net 6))
 (segment (start 102.099 139.128223) (end 102.099 127.651) (width 0.5) (layer "F.Cu") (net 6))
 (segment (start 102.099 127.651) (end 104 125.75) (width 0.5) (layer "F.Cu") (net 6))
 (segment (start 110.25 138) (end 110.25 138.04) (width 0.5) (layer "F.Cu") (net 6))
 (segment (start 110.25 138.04) (end 108.04 140.25) (width 0.5) (layer "F.Cu") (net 6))
 (segment (start 104 125.75) (end 108.04 125.75) (width 0.5) (layer "F.Cu") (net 6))
 (segment (start 104 140) (end 103 140) (width 0.5) (layer "F.Cu") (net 6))
 (via (at 111.858469 136.813681) (size 0.6) (drill 0.3) (layers "F.Cu" "B.Cu") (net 6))
 (segment (start 111.858469 136.813681) (end 111.5158 137.15635) (width 0.5) (layer "B.Cu") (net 6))
 (segment (start 111.5158 137.15635) (end 111.5158 137.912252) (width 0.5) (layer "B.Cu") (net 6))
 (segment (start 111.5158 137.912252) (end 111.9084 138.304852) (width 0.5) (layer "B.Cu") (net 6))
 (segment (start 117.073197 136.995001) (end 116.374999 136.995001) (width 0.2) (layer "F.Cu") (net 10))
 (segment (start 116.374999 136.995001) (end 115.33 138.04) (width 0.2) (layer "F.Cu") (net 10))
 (segment (start 115.33 127.96) (end 116.374999 129.004999) (width 0.2) (layer "F.Cu") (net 10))
 (segment (start 114.271385 126.901385) (end 115.33 127.96) (width 0.5) (layer "F.Cu") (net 10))
 (segment (start 116.374999 129.004999) (end 116.823197 129.004999) (width 0.2) (layer "F.Cu") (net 10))
 (segment (start 117.725 136.343198) (end 117.073197 136.995001) (width 0.2) (layer "F.Cu") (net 10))
 (segment (start 116.823197 129.004999) (end 117.725 129.906802) (width 0.2) (layer "F.Cu") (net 10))
 (segment (start 113.909277 126.901385) (end 114.271385 126.901385) (width 0.5) (layer "F.Cu") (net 10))
 (segment (start 117.725 129.906802) (end 117.725 136.343198) (width 0.2) (layer "F.Cu") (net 10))
 (via (at 113.909277 126.901385) (size 0.6) (drill 0.3) (layers "F.Cu" "B.Cu") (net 10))
 (segment (start 111.9084 128.8416) (end 113.848615 126.901385) (width 0.5) (layer "B.Cu") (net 10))
 (segment (start 113.848615 126.901385) (end 113.909277 126.901385) (width 0.5) (layer "B.Cu") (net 10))
 (segment (start 111.9084 129.604849) (end 111.9084 128.8416) (width 0.5) (layer "B.Cu") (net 10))
 (segment (start 117.275 130.093198) (end 117.275 136.156802) (width 0.2) (layer "F.Cu") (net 9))
 (segment (start 115.33 130.5) (end 116.374999 129.455001) (width 0.2) (layer "F.Cu") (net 9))
 (segment (start 116.636803 129.455001) (end 117.275 130.093198) (width 0.2) (layer "F.Cu") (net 9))
 (segment (start 114.25 129.25) (end 114.25 129.42) (width 0.5) (layer "F.Cu") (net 9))
 (segment (start 116.374999 136.544999) (end 115.33 135.5) (width 0.2) (layer "F.Cu") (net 9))
 (segment (start 114.25 129.42) (end 115.33 130.5) (width 0.5) (layer "F.Cu") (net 9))
 (segment (start 117.275 136.156802) (end 116.886803 136.544999) (width 0.2) (layer "F.Cu") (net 9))
 (segment (start 116.886803 136.544999) (end 116.374999 136.544999) (width 0.2) (layer "F.Cu") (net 9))
 (segment (start 116.374999 129.455001) (end 116.636803 129.455001) (width 0.2) (layer "F.Cu") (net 9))
 (via (at 114.25 129.25) (size 0.6) (drill 0.3) (layers "F.Cu" "B.Cu") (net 9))
 (segment (start 113.1584 129.604849) (end 113.895151 129.604849) (width 0.5) (layer "B.Cu") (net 9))
 (segment (start 113.895151 129.604849) (end 114.25 129.25) (width 0.5) (layer "B.Cu") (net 9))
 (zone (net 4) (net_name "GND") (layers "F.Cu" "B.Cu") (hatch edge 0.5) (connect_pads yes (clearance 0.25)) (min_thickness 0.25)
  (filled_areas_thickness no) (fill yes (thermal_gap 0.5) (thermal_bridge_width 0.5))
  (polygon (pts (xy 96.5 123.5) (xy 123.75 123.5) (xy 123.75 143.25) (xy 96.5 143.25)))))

